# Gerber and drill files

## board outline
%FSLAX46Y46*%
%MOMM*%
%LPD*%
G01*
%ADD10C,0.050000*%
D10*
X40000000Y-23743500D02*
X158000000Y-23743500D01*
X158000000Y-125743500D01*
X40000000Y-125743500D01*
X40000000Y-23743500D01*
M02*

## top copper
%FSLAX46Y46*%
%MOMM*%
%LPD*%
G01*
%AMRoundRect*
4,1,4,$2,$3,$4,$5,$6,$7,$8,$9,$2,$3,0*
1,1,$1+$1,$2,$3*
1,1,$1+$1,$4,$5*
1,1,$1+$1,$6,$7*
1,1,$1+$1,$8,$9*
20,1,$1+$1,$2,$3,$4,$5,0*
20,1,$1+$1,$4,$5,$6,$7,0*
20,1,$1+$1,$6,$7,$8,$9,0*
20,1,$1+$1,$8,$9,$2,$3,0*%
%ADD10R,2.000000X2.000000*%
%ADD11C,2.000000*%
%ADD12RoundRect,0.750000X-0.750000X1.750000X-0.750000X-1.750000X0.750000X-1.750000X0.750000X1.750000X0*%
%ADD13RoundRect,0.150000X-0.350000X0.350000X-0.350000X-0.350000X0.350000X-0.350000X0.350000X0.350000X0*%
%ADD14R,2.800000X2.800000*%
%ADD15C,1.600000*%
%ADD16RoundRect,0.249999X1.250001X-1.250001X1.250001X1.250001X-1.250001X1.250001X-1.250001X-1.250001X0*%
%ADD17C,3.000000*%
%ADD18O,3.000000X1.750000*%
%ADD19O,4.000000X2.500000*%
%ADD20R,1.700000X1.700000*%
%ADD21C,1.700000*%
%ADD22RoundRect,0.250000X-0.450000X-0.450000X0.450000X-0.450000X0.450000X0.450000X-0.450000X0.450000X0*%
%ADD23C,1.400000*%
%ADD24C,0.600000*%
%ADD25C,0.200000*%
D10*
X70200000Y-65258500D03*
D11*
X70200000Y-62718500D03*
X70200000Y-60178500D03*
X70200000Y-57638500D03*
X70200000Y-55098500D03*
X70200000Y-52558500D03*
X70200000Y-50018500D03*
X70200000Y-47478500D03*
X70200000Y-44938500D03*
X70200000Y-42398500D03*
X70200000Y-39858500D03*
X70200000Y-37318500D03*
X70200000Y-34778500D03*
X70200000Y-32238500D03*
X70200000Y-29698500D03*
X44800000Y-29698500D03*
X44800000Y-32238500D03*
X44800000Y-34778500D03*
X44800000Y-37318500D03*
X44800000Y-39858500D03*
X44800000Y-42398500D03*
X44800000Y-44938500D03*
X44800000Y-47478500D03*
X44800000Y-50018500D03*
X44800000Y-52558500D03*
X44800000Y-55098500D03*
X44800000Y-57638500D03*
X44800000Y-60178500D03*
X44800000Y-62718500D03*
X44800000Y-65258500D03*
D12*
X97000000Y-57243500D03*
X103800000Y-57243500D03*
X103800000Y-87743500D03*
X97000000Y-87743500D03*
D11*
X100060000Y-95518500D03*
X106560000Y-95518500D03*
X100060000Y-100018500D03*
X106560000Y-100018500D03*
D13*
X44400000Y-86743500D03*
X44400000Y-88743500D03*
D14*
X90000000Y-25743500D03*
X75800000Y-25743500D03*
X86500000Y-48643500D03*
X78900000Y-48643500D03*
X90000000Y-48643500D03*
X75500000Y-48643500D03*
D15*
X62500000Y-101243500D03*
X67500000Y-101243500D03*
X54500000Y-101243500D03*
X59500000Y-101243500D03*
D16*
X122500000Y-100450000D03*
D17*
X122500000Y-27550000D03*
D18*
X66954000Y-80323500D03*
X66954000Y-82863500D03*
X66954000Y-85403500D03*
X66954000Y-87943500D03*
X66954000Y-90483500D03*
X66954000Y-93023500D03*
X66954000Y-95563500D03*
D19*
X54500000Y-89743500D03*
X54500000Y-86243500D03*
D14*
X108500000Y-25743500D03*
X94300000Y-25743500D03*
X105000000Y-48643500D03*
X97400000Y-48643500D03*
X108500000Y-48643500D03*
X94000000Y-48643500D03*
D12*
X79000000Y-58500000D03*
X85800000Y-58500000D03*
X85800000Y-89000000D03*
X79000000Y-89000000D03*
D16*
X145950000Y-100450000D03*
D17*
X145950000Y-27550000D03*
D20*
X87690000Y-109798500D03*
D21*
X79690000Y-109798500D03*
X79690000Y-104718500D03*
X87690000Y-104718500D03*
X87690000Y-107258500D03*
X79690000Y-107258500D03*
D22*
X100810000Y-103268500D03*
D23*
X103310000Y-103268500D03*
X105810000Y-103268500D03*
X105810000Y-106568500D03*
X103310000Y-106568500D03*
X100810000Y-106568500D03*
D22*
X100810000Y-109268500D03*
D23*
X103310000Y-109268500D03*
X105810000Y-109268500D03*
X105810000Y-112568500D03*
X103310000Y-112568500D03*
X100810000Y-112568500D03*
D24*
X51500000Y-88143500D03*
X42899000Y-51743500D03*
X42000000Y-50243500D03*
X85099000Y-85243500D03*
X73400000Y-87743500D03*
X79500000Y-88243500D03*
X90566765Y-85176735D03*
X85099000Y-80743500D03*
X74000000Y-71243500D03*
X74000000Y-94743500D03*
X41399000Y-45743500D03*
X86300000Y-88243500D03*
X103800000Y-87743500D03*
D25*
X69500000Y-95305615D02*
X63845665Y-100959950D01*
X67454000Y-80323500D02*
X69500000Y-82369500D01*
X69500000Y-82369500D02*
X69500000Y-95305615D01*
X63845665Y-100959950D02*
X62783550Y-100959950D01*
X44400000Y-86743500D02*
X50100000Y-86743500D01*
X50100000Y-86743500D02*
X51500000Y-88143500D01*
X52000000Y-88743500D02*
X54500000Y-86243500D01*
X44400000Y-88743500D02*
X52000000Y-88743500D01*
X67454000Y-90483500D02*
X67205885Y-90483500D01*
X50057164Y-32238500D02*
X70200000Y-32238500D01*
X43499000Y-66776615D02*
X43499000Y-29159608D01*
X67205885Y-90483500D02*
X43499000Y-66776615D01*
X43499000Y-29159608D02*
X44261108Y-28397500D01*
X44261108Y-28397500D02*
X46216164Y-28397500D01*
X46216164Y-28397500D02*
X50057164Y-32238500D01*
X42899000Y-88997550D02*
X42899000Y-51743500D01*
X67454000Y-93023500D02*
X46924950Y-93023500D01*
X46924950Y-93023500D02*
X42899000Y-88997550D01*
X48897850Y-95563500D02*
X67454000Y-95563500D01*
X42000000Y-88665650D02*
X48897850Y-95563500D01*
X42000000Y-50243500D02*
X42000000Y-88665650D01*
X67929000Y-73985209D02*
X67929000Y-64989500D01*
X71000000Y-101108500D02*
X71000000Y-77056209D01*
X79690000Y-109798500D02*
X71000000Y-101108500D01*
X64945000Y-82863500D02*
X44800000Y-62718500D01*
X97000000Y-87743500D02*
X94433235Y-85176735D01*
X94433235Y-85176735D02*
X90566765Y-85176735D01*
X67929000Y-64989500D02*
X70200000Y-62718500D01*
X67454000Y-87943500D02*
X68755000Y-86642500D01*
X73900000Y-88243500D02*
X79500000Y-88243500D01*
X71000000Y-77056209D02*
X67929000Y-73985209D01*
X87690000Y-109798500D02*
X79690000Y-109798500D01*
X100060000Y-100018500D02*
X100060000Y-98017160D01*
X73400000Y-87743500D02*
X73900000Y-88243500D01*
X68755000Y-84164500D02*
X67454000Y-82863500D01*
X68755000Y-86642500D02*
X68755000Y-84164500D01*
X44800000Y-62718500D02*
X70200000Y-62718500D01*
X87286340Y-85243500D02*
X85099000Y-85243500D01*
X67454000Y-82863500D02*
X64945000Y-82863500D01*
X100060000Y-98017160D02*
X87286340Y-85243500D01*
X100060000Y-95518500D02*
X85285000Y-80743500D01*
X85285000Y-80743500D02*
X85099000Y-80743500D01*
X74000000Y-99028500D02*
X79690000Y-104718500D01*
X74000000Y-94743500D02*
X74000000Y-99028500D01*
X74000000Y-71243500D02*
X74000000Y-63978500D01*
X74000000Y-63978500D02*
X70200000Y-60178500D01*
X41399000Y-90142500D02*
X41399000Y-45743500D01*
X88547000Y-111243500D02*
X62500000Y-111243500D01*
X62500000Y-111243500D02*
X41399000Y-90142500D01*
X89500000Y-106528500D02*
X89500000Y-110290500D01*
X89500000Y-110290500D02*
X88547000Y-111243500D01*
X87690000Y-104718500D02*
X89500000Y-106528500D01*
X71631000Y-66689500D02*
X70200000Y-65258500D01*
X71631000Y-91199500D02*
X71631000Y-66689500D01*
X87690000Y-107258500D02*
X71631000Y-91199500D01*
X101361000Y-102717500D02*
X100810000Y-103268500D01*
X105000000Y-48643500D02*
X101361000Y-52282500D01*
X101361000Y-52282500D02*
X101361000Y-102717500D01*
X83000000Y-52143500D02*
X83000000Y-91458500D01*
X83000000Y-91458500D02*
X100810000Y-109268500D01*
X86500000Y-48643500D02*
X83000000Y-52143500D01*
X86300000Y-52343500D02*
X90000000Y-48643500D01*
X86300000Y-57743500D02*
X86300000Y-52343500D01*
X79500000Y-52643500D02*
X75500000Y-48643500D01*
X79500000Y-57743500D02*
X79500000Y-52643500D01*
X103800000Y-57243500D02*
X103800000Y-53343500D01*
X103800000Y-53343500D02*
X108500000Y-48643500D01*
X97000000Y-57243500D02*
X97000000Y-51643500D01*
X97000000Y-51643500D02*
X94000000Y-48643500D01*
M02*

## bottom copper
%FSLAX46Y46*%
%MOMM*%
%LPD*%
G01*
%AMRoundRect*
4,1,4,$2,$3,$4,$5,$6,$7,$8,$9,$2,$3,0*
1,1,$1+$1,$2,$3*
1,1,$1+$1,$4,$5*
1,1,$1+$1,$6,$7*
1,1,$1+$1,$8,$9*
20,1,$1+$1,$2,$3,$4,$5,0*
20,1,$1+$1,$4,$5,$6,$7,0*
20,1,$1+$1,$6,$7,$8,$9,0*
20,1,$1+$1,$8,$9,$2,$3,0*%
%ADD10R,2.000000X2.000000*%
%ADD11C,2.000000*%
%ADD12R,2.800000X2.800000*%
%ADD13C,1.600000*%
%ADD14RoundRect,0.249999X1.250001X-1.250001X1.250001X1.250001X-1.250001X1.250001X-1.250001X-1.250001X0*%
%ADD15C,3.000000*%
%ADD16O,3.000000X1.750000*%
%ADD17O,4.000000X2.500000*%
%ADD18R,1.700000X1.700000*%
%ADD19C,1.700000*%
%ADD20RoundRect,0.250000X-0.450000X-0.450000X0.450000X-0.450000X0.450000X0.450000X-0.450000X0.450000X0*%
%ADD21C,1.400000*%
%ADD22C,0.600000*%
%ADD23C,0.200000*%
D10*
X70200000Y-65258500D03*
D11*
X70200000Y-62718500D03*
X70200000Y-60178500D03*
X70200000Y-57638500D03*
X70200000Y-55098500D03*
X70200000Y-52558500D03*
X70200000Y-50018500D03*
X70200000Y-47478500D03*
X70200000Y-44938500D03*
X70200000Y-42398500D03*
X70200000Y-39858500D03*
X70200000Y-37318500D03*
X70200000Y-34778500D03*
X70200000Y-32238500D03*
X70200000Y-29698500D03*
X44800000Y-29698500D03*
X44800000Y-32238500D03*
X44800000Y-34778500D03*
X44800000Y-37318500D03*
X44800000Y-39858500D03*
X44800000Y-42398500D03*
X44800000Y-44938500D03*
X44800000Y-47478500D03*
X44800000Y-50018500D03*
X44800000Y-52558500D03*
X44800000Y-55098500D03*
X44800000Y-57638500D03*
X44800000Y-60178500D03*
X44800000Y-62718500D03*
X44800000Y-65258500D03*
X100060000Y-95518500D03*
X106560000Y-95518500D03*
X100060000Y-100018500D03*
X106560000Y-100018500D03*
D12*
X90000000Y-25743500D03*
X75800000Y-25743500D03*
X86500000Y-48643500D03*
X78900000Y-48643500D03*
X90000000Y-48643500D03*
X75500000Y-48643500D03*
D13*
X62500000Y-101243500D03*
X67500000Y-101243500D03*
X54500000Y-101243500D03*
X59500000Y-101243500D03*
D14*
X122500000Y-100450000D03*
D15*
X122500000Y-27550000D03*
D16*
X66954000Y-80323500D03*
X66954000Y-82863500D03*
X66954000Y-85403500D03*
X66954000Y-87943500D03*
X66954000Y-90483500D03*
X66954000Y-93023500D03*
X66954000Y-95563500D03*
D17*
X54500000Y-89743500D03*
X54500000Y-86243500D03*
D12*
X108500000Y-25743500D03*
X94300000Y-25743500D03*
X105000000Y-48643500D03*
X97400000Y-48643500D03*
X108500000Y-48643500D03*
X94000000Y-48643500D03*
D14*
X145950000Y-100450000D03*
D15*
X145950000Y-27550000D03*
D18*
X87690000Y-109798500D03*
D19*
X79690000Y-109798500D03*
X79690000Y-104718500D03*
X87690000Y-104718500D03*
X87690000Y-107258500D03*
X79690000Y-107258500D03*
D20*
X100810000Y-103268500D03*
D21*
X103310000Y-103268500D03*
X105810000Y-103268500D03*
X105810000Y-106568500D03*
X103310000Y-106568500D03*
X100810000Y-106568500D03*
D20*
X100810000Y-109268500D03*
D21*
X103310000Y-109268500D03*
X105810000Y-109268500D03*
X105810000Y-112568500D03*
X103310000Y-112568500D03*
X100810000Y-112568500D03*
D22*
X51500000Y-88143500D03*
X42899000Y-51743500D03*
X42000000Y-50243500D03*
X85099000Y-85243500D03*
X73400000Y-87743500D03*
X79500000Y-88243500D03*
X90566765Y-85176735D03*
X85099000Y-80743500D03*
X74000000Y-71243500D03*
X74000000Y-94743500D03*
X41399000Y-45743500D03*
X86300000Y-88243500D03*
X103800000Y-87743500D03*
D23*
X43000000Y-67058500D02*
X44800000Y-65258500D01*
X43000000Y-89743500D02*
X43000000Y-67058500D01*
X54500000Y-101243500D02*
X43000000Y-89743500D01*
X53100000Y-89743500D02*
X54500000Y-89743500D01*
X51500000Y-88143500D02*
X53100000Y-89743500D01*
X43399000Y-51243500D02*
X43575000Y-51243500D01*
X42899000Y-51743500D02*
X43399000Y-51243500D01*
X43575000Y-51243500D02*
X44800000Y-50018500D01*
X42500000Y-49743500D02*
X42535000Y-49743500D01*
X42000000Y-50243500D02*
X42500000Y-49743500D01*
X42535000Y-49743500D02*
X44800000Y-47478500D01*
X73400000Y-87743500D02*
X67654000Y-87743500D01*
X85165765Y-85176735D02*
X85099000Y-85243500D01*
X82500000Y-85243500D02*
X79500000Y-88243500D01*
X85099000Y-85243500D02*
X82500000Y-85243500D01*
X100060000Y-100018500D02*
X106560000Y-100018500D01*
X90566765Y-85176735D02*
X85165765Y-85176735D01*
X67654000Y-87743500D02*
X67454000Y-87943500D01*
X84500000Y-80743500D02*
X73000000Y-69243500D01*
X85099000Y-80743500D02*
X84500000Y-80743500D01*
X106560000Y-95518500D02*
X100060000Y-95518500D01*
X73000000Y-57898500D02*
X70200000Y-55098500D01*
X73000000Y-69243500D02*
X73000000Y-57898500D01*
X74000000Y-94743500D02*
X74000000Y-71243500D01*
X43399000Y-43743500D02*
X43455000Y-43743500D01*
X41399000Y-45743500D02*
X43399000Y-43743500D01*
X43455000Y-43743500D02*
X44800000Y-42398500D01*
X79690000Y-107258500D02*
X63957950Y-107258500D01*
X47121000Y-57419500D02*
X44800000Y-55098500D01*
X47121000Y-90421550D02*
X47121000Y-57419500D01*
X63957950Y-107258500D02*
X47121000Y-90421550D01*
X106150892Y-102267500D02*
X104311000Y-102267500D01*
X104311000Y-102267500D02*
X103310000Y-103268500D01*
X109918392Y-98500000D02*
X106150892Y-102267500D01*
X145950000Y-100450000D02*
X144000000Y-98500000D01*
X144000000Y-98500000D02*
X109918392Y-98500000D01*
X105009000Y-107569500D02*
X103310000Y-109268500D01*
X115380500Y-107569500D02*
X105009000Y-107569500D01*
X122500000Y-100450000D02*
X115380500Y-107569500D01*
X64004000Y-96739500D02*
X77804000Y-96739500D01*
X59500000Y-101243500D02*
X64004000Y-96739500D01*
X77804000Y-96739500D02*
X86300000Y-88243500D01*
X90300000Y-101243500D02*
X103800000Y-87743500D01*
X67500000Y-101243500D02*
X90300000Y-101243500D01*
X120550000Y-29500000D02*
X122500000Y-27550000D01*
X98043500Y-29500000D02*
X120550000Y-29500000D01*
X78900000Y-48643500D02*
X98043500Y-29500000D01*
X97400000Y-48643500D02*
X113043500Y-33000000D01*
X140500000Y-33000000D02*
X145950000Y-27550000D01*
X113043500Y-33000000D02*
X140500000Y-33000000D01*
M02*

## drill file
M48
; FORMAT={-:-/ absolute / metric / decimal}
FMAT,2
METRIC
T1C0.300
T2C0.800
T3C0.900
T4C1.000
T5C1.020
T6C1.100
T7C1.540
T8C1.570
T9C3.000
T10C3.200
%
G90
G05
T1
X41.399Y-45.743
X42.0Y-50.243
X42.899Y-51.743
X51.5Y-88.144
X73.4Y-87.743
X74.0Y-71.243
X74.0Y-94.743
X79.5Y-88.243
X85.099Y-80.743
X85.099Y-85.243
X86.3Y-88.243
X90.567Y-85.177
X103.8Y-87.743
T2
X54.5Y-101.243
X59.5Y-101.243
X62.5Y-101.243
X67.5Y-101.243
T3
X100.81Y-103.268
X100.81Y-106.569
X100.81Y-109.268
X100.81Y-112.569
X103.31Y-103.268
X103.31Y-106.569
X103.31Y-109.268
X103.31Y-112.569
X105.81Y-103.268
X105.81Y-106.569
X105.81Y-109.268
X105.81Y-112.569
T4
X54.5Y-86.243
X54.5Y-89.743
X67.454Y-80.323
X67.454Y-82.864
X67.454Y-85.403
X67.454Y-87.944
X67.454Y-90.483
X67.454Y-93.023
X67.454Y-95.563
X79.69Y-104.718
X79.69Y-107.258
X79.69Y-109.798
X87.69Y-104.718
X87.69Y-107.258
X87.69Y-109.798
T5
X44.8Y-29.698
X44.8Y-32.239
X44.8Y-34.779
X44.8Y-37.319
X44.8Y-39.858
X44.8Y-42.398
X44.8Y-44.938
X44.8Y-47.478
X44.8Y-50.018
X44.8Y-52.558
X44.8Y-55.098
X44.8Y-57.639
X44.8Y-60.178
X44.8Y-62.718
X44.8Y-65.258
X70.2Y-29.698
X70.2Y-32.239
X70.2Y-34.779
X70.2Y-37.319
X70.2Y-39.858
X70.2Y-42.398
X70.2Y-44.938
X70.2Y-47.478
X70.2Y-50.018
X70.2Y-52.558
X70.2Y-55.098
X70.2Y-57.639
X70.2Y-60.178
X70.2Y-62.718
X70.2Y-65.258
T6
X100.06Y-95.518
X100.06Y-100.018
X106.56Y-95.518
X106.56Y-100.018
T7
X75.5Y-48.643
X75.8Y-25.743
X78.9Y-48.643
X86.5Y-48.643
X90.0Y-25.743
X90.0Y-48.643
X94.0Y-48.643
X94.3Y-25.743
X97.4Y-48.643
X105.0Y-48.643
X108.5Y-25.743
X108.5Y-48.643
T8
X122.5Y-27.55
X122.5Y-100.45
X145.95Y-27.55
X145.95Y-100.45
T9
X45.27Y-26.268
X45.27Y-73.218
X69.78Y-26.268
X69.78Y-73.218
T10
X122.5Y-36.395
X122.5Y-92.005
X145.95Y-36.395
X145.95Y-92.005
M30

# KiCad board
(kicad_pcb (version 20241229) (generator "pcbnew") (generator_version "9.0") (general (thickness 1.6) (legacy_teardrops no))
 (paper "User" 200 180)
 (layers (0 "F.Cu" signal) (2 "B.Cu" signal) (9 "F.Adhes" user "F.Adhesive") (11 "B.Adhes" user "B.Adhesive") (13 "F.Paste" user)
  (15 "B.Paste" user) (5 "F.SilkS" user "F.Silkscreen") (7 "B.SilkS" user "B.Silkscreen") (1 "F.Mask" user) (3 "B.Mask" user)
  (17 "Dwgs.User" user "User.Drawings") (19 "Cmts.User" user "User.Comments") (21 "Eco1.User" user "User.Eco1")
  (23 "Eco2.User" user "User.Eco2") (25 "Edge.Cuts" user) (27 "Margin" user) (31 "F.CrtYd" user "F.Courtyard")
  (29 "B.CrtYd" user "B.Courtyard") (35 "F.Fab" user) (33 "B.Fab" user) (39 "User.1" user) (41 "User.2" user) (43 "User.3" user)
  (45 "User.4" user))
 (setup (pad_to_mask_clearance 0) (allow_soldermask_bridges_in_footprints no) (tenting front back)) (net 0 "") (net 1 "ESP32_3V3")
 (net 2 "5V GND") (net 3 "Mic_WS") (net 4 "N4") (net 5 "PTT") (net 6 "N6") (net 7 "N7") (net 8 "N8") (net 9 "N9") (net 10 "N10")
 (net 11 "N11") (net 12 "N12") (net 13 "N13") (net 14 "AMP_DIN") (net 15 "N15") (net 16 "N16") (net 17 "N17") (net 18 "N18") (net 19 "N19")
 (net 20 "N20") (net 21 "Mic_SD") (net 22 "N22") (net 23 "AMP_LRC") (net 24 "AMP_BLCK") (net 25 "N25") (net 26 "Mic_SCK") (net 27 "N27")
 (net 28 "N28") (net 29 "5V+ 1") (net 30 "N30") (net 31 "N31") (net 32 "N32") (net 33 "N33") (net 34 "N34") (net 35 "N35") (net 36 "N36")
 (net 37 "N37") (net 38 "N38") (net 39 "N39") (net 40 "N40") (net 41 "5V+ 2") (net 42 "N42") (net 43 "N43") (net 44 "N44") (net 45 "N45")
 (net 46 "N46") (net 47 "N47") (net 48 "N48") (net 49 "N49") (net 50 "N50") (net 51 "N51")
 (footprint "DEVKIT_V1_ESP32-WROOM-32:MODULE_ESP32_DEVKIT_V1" (layer "F.Cu") (at 57.5 49.7435 180)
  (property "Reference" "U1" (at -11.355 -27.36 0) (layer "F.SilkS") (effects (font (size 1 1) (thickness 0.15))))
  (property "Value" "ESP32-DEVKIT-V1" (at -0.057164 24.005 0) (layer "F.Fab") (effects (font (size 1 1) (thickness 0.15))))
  (pad "" np_thru_hole circle (at -12.28 -23.475 180) (size 3 3) (drill 3) (layers "*.Cu" "*.Mask"))
  (pad "" np_thru_hole circle (at -12.28 23.475 180) (size 3 3) (drill 3) (layers "*.Cu" "*.Mask"))
  (pad "" np_thru_hole circle (at 12.23 -23.475 180) (size 3 3) (drill 3) (layers "*.Cu" "*.Mask"))
  (pad "" np_thru_hole circle (at 12.23 23.475 180) (size 3 3) (drill 3) (layers "*.Cu" "*.Mask"))
  (pad "1" thru_hole rect (at -12.7 -15.515 180) (size 2 2) (drill 1.02) (layers "*.Cu" "*.Mask") (remove_unused_layers no)
   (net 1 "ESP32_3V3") (solder_mask_margin 0.102))
  (pad "2" thru_hole circle (at -12.7 -12.975 180) (size 2 2) (drill 1.02) (layers "*.Cu" "*.Mask") (remove_unused_layers no)
   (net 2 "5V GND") (solder_mask_margin 0.102))
  (pad "3" thru_hole circle (at -12.7 -10.435 180) (size 2 2) (drill 1.02) (layers "*.Cu" "*.Mask") (remove_unused_layers no)
   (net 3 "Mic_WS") (solder_mask_margin 0.102))
  (pad "4" thru_hole circle (at -12.7 -7.895 180) (size 2 2) (drill 1.02) (layers "*.Cu" "*.Mask") (remove_unused_layers no) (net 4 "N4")
   (solder_mask_margin 0.102))
  (pad "5" thru_hole circle (at -12.7 -5.355 180) (size 2 2) (drill 1.02) (layers "*.Cu" "*.Mask") (remove_unused_layers no) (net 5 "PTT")
   (solder_mask_margin 0.102))
  (pad "6" thru_hole circle (at -12.7 -2.815 180) (size 2 2) (drill 1.02) (layers "*.Cu" "*.Mask") (remove_unused_layers no) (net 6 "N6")
   (solder_mask_margin 0.102))
  (pad "7" thru_hole circle (at -12.7 -0.275 180) (size 2 2) (drill 1.02) (layers "*.Cu" "*.Mask") (remove_unused_layers no) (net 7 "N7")
   (solder_mask_margin 0.102))
  (pad "8" thru_hole circle (at -12.7 2.265 180) (size 2 2) (drill 1.02) (layers "*.Cu" "*.Mask") (remove_unused_layers no) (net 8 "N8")
   (solder_mask_margin 0.102))
  (pad "9" thru_hole circle (at -12.7 4.805 180) (size 2 2) (drill 1.02) (layers "*.Cu" "*.Mask") (remove_unused_layers no) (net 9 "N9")
   (solder_mask_margin 0.102))
  (pad "10" thru_hole circle (at -12.7 7.345 180) (size 2 2) (drill 1.02) (layers "*.Cu" "*.Mask") (remove_unused_layers no) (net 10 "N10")
   (solder_mask_margin 0.102))
  (pad "11" thru_hole circle (at -12.7 9.885 180) (size 2 2) (drill 1.02) (layers "*.Cu" "*.Mask") (remove_unused_layers no) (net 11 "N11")
   (solder_mask_margin 0.102))
  (pad "12" thru_hole circle (at -12.7 12.425 180) (size 2 2) (drill 1.02) (layers "*.Cu" "*.Mask") (remove_unused_layers no) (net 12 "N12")
   (solder_mask_margin 0.102))
  (pad "13" thru_hole circle (at -12.7 14.965 180) (size 2 2) (drill 1.02) (layers "*.Cu" "*.Mask") (remove_unused_layers no) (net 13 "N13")
   (solder_mask_margin 0.102))
  (pad "14" thru_hole circle (at -12.7 17.505 180) (size 2 2) (drill 1.02) (layers "*.Cu" "*.Mask") (remove_unused_layers no)
   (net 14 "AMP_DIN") (solder_mask_margin 0.102))
  (pad "15" thru_hole circle (at -12.7 20.045 180) (size 2 2) (drill 1.02) (layers "*.Cu" "*.Mask") (remove_unused_layers no) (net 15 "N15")
   (solder_mask_margin 0.102))
  (pad "16" thru_hole circle (at 12.7 20.045 180) (size 2 2) (drill 1.02) (layers "*.Cu" "*.Mask") (remove_unused_layers no) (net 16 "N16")
   (solder_mask_margin 0.102))
  (pad "17" thru_hole circle (at 12.7 17.505 180) (size 2 2) (drill 1.02) (layers "*.Cu" "*.Mask") (remove_unused_layers no) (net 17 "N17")
   (solder_mask_margin 0.102))
  (pad "18" thru_hole circle (at 12.7 14.965 180) (size 2 2) (drill 1.02) (layers "*.Cu" "*.Mask") (remove_unused_layers no) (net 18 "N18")
   (solder_mask_margin 0.102))
  (pad "19" thru_hole circle (at 12.7 12.425 180) (size 2 2) (drill 1.02) (layers "*.Cu" "*.Mask") (remove_unused_layers no) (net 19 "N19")
   (solder_mask_margin 0.102))
  (pad "20" thru_hole circle (at 12.7 9.885 180) (size 2 2) (drill 1.02) (layers "*.Cu" "*.Mask") (remove_unused_layers no) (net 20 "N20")
   (solder_mask_margin 0.102))
  (pad "21" thru_hole circle (at 12.7 7.345 180) (size 2 2) (drill 1.02) (layers "*.Cu" "*.Mask") (remove_unused_layers no)
   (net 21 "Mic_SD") (solder_mask_margin 0.102))
  (pad "22" thru_hole circle (at 12.7 4.805 180) (size 2 2) (drill 1.02) (layers "*.Cu" "*.Mask") (remove_unused_layers no) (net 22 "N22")
   (solder_mask_margin 0.102))
  (pad "23" thru_hole circle (at 12.7 2.265 180) (size 2 2) (drill 1.02) (layers "*.Cu" "*.Mask") (remove_unused_layers no)
   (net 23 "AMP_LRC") (solder_mask_margin 0.102))
  (pad "24" thru_hole circle (at 12.7 -0.275 180) (size 2 2) (drill 1.02) (layers "*.Cu" "*.Mask") (remove_unused_layers no)
   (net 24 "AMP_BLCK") (solder_mask_margin 0.102))
  (pad "25" thru_hole circle (at 12.7 -2.815 180) (size 2 2) (drill 1.02) (layers "*.Cu" "*.Mask") (remove_unused_layers no) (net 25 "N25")
   (solder_mask_margin 0.102))
  (pad "26" thru_hole circle (at 12.7 -5.355 180) (size 2 2) (drill 1.02) (layers "*.Cu" "*.Mask") (remove_unused_layers no)
   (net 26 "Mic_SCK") (solder_mask_margin 0.102))
  (pad "27" thru_hole circle (at 12.7 -7.895 180) (size 2 2) (drill 1.02) (layers "*.Cu" "*.Mask") (remove_unused_layers no) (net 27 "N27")
   (solder_mask_margin 0.102))
  (pad "28" thru_hole circle (at 12.7 -10.435 180) (size 2 2) (drill 1.02) (layers "*.Cu" "*.Mask") (remove_unused_layers no) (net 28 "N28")
   (solder_mask_margin 0.102))
  (pad "29" thru_hole circle (at 12.7 -12.975 180) (size 2 2) (drill 1.02) (layers "*.Cu" "*.Mask") (remove_unused_layers no)
   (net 2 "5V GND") (solder_mask_margin 0.102))
  (pad "30" thru_hole circle (at 12.7 -15.515 180) (size 2 2) (drill 1.02) (layers "*.Cu" "*.Mask") (remove_unused_layers no)
   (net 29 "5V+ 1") (solder_mask_margin 0.102))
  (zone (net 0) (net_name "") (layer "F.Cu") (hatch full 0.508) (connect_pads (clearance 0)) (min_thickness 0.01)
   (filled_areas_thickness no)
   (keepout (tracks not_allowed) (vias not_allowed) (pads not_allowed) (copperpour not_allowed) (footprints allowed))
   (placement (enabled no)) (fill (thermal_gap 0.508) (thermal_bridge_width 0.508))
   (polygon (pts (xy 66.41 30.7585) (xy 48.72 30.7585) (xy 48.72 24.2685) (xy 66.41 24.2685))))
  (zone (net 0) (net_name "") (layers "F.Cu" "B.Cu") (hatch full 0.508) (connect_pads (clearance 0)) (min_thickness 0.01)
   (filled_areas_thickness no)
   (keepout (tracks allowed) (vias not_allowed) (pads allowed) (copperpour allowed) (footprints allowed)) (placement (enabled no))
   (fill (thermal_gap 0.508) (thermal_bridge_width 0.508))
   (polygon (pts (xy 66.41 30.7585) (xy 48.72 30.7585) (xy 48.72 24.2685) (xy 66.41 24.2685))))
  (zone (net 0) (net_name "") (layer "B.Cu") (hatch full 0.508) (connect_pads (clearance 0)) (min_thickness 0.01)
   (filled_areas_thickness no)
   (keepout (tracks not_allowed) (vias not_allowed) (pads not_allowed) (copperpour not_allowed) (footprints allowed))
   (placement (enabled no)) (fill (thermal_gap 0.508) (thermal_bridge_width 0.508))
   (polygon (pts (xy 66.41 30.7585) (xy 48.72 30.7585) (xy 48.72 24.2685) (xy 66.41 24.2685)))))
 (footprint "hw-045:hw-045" (layer "F.Cu") (at 99.9 72.2435 -90)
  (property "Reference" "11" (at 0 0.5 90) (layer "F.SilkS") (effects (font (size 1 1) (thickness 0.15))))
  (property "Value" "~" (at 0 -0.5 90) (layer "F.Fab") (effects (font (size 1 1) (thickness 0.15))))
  (pad "1" smd roundrect (at -15 2.9 270) (size 5 3) (layers "F.Cu" "F.Mask" "F.Paste") (roundrect_rratio 0.25) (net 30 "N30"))
  (pad "2" smd roundrect (at -15 -3.9 270) (size 5 3) (layers "F.Cu" "F.Mask" "F.Paste") (roundrect_rratio 0.25) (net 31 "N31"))
  (pad "3" smd roundrect (at 15.5 -3.9 270) (size 5 3) (layers "F.Cu" "F.Mask" "F.Paste") (roundrect_rratio 0.25) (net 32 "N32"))
  (pad "4" smd roundrect (at 15.5 2.9 270) (size 5 3) (layers "F.Cu" "F.Mask" "F.Paste") (roundrect_rratio 0.25) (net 2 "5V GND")))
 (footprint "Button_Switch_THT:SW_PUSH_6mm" (layer "F.Cu") (at 100.06 95.5185)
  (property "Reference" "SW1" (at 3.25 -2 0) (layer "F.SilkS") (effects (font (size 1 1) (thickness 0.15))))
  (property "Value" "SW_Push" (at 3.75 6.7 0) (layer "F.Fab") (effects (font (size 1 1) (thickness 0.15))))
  (pad "1" thru_hole circle (at 0 0 90) (size 2 2) (drill 1.1) (layers "*.Cu" "*.Mask") (remove_unused_layers no) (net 5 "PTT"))
  (pad "1" thru_hole circle (at 6.5 0 90) (size 2 2) (drill 1.1) (layers "*.Cu" "*.Mask") (remove_unused_layers no) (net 5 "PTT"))
  (pad "2" thru_hole circle (at 0 4.5 90) (size 2 2) (drill 1.1) (layers "*.Cu" "*.Mask") (remove_unused_layers no) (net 2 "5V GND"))
  (pad "2" thru_hole circle (at 6.5 4.5 90) (size 2 2) (drill 1.1) (layers "*.Cu" "*.Mask") (remove_unused_layers no) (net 2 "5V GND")))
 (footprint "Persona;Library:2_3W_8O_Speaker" (layer "F.Cu") (at 45.4 87.7435 -90)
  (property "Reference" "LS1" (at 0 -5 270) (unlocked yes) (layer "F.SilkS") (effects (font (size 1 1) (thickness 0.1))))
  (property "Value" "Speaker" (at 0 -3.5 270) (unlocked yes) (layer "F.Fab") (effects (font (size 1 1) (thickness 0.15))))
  (pad "1" smd roundrect (at -1 1 270) (size 1 1) (layers "F.Cu" "F.Mask" "F.Paste") (roundrect_rratio 0.15) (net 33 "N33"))
  (pad "2" smd roundrect (at 1 1 270) (size 1 1) (layers "F.Cu" "F.Mask" "F.Paste") (roundrect_rratio 0.15) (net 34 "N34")))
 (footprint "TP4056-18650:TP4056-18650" (layer "F.Cu") (at 91.7 24.0435 -90)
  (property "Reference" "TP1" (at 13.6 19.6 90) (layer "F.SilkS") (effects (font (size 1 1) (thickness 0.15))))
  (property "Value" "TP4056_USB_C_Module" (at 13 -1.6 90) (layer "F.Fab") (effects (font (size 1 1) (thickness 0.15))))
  (pad "1" thru_hole rect (at 1.7 1.7 270) (size 2.8 2.8) (drill 1.54) (layers "*.Cu" "*.Mask") (remove_unused_layers no) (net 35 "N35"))
  (pad "2" thru_hole rect (at 1.7 15.9 270) (size 2.8 2.8) (drill 1.54) (layers "*.Cu" "*.Mask") (remove_unused_layers no) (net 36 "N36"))
  (pad "3" thru_hole rect (at 24.6 5.2 270) (size 2.8 2.8) (drill 1.54) (layers "*.Cu" "*.Mask") (remove_unused_layers no) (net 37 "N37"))
  (pad "4" thru_hole rect (at 24.6 12.8 270) (size 2.8 2.8) (drill 1.54) (layers "*.Cu" "*.Mask") (remove_unused_layers no) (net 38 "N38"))
  (pad "5" thru_hole rect (at 24.6 1.7 270) (size 2.8 2.8) (drill 1.54) (layers "*.Cu" "*.Mask") (remove_unused_layers no) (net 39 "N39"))
  (pad "6" thru_hole rect (at 24.6 16.2 270) (size 2.8 2.8) (drill 1.54) (layers "*.Cu" "*.Mask") (remove_unused_layers no) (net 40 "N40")))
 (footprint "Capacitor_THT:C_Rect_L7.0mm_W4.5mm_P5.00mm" (layer "F.Cu") (at 62.5 101.2435)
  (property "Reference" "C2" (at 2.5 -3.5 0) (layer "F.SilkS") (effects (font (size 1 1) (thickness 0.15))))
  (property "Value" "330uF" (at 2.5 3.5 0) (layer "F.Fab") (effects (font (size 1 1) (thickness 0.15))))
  (pad "1" thru_hole circle (at 0 0) (size 1.6 1.6) (drill 0.8) (layers "*.Cu" "*.Mask") (remove_unused_layers no) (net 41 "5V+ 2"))
  (pad "2" thru_hole circle (at 5 0) (size 1.6 1.6) (drill 0.8) (layers "*.Cu" "*.Mask") (remove_unused_layers no) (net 32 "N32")))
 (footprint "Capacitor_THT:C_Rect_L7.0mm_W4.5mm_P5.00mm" (layer "F.Cu") (at 54.5 101.2435)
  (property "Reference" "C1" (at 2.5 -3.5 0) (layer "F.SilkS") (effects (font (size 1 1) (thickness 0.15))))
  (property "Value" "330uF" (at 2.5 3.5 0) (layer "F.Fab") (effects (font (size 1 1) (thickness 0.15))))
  (pad "1" thru_hole circle (at 0 0) (size 1.6 1.6) (drill 0.8) (layers "*.Cu" "*.Mask") (remove_unused_layers no) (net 29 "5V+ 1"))
  (pad "2" thru_hole circle (at 5 0) (size 1.6 1.6) (drill 0.8) (layers "*.Cu" "*.Mask") (remove_unused_layers no) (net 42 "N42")))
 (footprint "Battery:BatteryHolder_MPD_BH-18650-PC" (layer "F.Cu") (at 122.5 100.45 90)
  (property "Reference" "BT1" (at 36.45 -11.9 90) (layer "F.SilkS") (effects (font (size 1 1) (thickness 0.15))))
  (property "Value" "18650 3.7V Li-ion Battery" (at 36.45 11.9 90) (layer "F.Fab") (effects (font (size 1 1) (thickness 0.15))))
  (pad "" np_thru_hole circle (at 8.445 0 90) (size 3.2 3.2) (drill 3.2) (layers "*.Cu" "*.Mask"))
  (pad "" np_thru_hole circle (at 64.055 0 90) (size 3.2 3.2) (drill 3.2) (layers "*.Cu" "*.Mask"))
  (pad "1" thru_hole roundrect (at 0 0 90) (size 3 3) (drill 1.57) (layers "*.Cu" "*.Mask") (remove_unused_layers no)
   (roundrect_rratio 0.083333) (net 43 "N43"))
  (pad "2" thru_hole circle (at 72.9 0 90) (size 3 3) (drill 1.57) (layers "*.Cu" "*.Mask") (remove_unused_layers no) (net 38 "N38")))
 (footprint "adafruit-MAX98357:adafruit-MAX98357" (layer "F.Cu") (at 60.547 87.8235 90)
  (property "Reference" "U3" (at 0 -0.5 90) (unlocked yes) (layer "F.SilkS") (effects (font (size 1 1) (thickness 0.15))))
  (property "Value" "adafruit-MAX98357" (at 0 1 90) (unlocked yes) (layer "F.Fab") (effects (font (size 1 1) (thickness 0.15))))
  (pad "1" thru_hole oval (at 7.5 6.907) (size 3 1.75) (drill 1 (offset -0.5 0)) (layers "*.Cu" "*.Mask") (remove_unused_layers no)
   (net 41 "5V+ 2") (solder_mask_margin 0.0508))
  (pad "2" thru_hole oval (at 4.96 6.907) (size 3 1.75) (drill 1 (offset -0.5 0)) (layers "*.Cu" "*.Mask") (remove_unused_layers no)
   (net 2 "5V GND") (solder_mask_margin 0.0508))
  (pad "3" thru_hole oval (at 2.42 6.907) (size 3 1.75) (drill 1 (offset -0.5 0)) (layers "*.Cu" "*.Mask") (remove_unused_layers no)
   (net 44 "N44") (solder_mask_margin 0.0508))
  (pad "4" thru_hole oval (at -0.12 6.907) (size 3 1.75) (drill 1 (offset -0.5 0)) (layers "*.Cu" "*.Mask") (remove_unused_layers no)
   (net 2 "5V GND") (solder_mask_margin 0.0508))
  (pad "5" thru_hole oval (at -2.66 6.907) (size 3 1.75) (drill 1 (offset -0.5 0)) (layers "*.Cu" "*.Mask") (remove_unused_layers no)
   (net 14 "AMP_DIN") (solder_mask_margin 0.0508))
  (pad "6" thru_hole oval (at -5.2 6.907) (size 3 1.75) (drill 1 (offset -0.5 0)) (layers "*.Cu" "*.Mask") (remove_unused_layers no)
   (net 24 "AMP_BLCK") (solder_mask_margin 0.0508))
  (pad "7" thru_hole oval (at -7.74 6.907) (size 3 1.75) (drill 1 (offset -0.5 0)) (layers "*.Cu" "*.Mask") (remove_unused_layers no)
   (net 23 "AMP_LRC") (solder_mask_margin 0.0508))
  (pad "8" thru_hole oval (at -1.92 -6.047 270) (size 2.5 4) (drill 1) (layers "*.Cu" "*.Mask") (remove_unused_layers no) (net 33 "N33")
   (solder_mask_margin 0.0508))
  (pad "9" thru_hole oval (at 1.58 -6.047 270) (size 2.5 4) (drill 1) (layers "*.Cu" "*.Mask") (remove_unused_layers no) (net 34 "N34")
   (solder_mask_margin 0.0508)))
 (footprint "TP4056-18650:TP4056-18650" (layer "F.Cu") (at 110.2 24.0435 -90)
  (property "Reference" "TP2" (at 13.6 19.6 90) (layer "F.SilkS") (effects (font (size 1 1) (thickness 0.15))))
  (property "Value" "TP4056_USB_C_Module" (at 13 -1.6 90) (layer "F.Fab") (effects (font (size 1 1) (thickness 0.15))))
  (pad "1" thru_hole rect (at 1.7 1.7 270) (size 2.8 2.8) (drill 1.54) (layers "*.Cu" "*.Mask") (remove_unused_layers no) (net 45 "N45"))
  (pad "2" thru_hole rect (at 1.7 15.9 270) (size 2.8 2.8) (drill 1.54) (layers "*.Cu" "*.Mask") (remove_unused_layers no) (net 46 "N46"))
  (pad "3" thru_hole rect (at 24.6 5.2 270) (size 2.8 2.8) (drill 1.54) (layers "*.Cu" "*.Mask") (remove_unused_layers no) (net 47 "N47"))
  (pad "4" thru_hole rect (at 24.6 12.8 270) (size 2.8 2.8) (drill 1.54) (layers "*.Cu" "*.Mask") (remove_unused_layers no) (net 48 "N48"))
  (pad "5" thru_hole rect (at 24.6 1.7 270) (size 2.8 2.8) (drill 1.54) (layers "*.Cu" "*.Mask") (remove_unused_layers no) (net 31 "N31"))
  (pad "6" thru_hole rect (at 24.6 16.2 270) (size 2.8 2.8) (drill 1.54) (layers "*.Cu" "*.Mask") (remove_unused_layers no) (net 30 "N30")))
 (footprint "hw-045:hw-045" (layer "F.Cu") (at 81.9 73.5 -90)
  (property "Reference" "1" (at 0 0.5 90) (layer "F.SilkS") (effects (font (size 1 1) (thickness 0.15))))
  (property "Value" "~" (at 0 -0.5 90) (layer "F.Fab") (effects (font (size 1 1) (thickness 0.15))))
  (pad "1" smd roundrect (at -15 2.9 270) (size 5 3) (layers "F.Cu" "F.Mask" "F.Paste") (roundrect_rratio 0.25) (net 40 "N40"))
  (pad "2" smd roundrect (at -15 -3.9 270) (size 5 3) (layers "F.Cu" "F.Mask" "F.Paste") (roundrect_rratio 0.25) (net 39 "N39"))
  (pad "3" smd roundrect (at 15.5 -3.9 270) (size 5 3) (layers "F.Cu" "F.Mask" "F.Paste") (roundrect_rratio 0.25) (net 42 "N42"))
  (pad "4" smd roundrect (at 15.5 2.9 270) (size 5 3) (layers "F.Cu" "F.Mask" "F.Paste") (roundrect_rratio 0.25) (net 2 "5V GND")))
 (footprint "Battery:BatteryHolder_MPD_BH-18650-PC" (layer "F.Cu") (at 145.95 100.45 90)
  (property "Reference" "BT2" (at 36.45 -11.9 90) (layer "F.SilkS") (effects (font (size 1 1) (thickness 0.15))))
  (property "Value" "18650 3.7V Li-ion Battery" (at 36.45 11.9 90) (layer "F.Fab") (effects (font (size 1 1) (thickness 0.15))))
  (pad "" np_thru_hole circle (at 8.445 0 90) (size 3.2 3.2) (drill 3.2) (layers "*.Cu" "*.Mask"))
  (pad "" np_thru_hole circle (at 64.055 0 90) (size 3.2 3.2) (drill 3.2) (layers "*.Cu" "*.Mask"))
  (pad "1" thru_hole roundrect (at 0 0 90) (size 3 3) (drill 1.57) (layers "*.Cu" "*.Mask") (remove_unused_layers no)
   (roundrect_rratio 0.083333) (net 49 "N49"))
  (pad "2" thru_hole circle (at 72.9 0 90) (size 3 3) (drill 1.57) (layers "*.Cu" "*.Mask") (remove_unused_layers no) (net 48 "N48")))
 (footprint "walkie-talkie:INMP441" (layer "F.Cu") (at 83.5 114.2435 180)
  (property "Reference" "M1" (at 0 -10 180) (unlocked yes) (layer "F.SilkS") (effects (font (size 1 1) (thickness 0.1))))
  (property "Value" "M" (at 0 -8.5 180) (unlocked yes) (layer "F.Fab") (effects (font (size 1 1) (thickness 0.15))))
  (pad "GND" thru_hole rect (at -4.19 4.445 180) (size 1.7 1.7) (drill 1) (layers "*.Cu" "*.Mask") (remove_unused_layers no)
   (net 2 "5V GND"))
  (pad "L/R" thru_hole circle (at 3.81 4.445 180) (size 1.7 1.7) (drill 1) (layers "*.Cu" "*.Mask") (remove_unused_layers no)
   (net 2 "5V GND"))
  (pad "SCK" thru_hole circle (at 3.81 9.525 180) (size 1.7 1.7) (drill 1) (layers "*.Cu" "*.Mask") (remove_unused_layers no)
   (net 3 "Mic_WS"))
  (pad "SD" thru_hole circle (at -4.19 9.525 180) (size 1.7 1.7) (drill 1) (layers "*.Cu" "*.Mask") (remove_unused_layers no)
   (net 21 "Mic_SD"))
  (pad "VDD" thru_hole circle (at -4.19 6.985 180) (size 1.7 1.7) (drill 1) (layers "*.Cu" "*.Mask") (remove_unused_layers no)
   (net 1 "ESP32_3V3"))
  (pad "WS" thru_hole circle (at 3.81 6.985 180) (size 1.7 1.7) (drill 1) (layers "*.Cu" "*.Mask") (remove_unused_layers no)
   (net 26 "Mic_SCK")))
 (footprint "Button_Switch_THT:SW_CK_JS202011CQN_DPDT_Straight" (layer "F.Cu") (at 100.81 103.2685)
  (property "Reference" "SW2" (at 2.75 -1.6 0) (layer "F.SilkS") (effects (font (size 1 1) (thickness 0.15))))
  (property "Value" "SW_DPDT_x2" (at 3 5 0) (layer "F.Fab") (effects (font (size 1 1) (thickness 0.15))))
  (pad "1" thru_hole roundrect (at 0 0) (size 1.4 1.4) (drill 0.9) (layers "*.Cu" "*.Mask") (remove_unused_layers no)
   (roundrect_rratio 0.1785714286) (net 47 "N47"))
  (pad "2" thru_hole circle (at 2.5 0) (size 1.4 1.4) (drill 0.9) (layers "*.Cu" "*.Mask") (remove_unused_layers no) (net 49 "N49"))
  (pad "3" thru_hole circle (at 5 0) (size 1.4 1.4) (drill 0.9) (layers "*.Cu" "*.Mask") (remove_unused_layers no) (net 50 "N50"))
  (pad "4" thru_hole circle (at 5 3.3) (size 1.4 1.4) (drill 0.9) (layers "*.Cu" "*.Mask") (remove_unused_layers no))
  (pad "5" thru_hole circle (at 2.5 3.3) (size 1.4 1.4) (drill 0.9) (layers "*.Cu" "*.Mask") (remove_unused_layers no))
  (pad "6" thru_hole circle (at 0 3.3) (size 1.4 1.4) (drill 0.9) (layers "*.Cu" "*.Mask") (remove_unused_layers no)))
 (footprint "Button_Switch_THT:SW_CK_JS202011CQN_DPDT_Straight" (layer "F.Cu") (at 100.81 109.2685)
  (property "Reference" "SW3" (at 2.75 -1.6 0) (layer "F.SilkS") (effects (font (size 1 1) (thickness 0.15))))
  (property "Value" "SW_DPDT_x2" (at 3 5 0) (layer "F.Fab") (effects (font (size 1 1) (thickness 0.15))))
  (pad "1" thru_hole roundrect (at 0 0) (size 1.4 1.4) (drill 0.9) (layers "*.Cu" "*.Mask") (remove_unused_layers no)
   (roundrect_rratio 0.1785714286) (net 37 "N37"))
  (pad "2" thru_hole circle (at 2.5 0) (size 1.4 1.4) (drill 0.9) (layers "*.Cu" "*.Mask") (remove_unused_layers no) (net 43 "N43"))
  (pad "3" thru_hole circle (at 5 0) (size 1.4 1.4) (drill 0.9) (layers "*.Cu" "*.Mask") (remove_unused_layers no) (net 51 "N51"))
  (pad "4" thru_hole circle (at 5 3.3) (size 1.4 1.4) (drill 0.9) (layers "*.Cu" "*.Mask") (remove_unused_layers no))
  (pad "5" thru_hole circle (at 2.5 3.3) (size 1.4 1.4) (drill 0.9) (layers "*.Cu" "*.Mask") (remove_unused_layers no))
  (pad "6" thru_hole circle (at 0 3.3) (size 1.4 1.4) (drill 0.9) (layers "*.Cu" "*.Mask") (remove_unused_layers no)))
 (gr_rect (start 40 23.7435) (end 158 125.7435) (stroke (width 0.05) (type default)) (fill no) (layer "Edge.Cuts"))
 (segment (start 43 67.0585) (end 44.8 65.2585) (width 0.2) (layer "B.Cu") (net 29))
 (segment (start 43 89.7435) (end 43 67.0585) (width 0.2) (layer "B.Cu") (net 29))
 (segment (start 54.5 101.2435) (end 43 89.7435) (width 0.2) (layer "B.Cu") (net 29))
 (segment (start 69.5 95.305615) (end 63.845665 100.95995) (width 0.2) (layer "F.Cu") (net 41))
 (segment (start 67.454 80.3235) (end 69.5 82.3695) (width 0.2) (layer "F.Cu") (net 41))
 (segment (start 69.5 82.3695) (end 69.5 95.305615) (width 0.2) (layer "F.Cu") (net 41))
 (segment (start 63.845665 100.95995) (end 62.78355 100.95995) (width 0.2) (layer "F.Cu") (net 41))
 (segment (start 44.4 86.7435) (end 50.1 86.7435) (width 0.2) (layer "F.Cu") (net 33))
 (segment (start 50.1 86.7435) (end 51.5 88.1435) (width 0.2) (layer "F.Cu") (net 33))
 (via (at 51.5 88.1435) (size 0.6) (drill 0.3) (layers "F.Cu" "B.Cu") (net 33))
 (segment (start 53.1 89.7435) (end 54.5 89.7435) (width 0.2) (layer "B.Cu") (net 33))
 (segment (start 51.5 88.1435) (end 53.1 89.7435) (width 0.2) (layer "B.Cu") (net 33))
 (segment (start 52 88.7435) (end 54.5 86.2435) (width 0.2) (layer "F.Cu") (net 34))
 (segment (start 44.4 88.7435) (end 52 88.7435) (width 0.2) (layer "F.Cu") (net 34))
 (segment (start 67.454 90.4835) (end 67.205885 90.4835) (width 0.2) (layer "F.Cu") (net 14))
 (segment (start 50.057164 32.2385) (end 70.2 32.2385) (width 0.2) (layer "F.Cu") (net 14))
 (segment (start 43.499 66.776615) (end 43.499 29.159608) (width 0.2) (layer "F.Cu") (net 14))
 (segment (start 67.205885 90.4835) (end 43.499 66.776615) (width 0.2) (layer "F.Cu") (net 14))
 (segment (start 43.499 29.159608) (end 44.261108 28.3975) (width 0.2) (layer "F.Cu") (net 14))
 (segment (start 44.261108 28.3975) (end 46.216164 28.3975) (width 0.2) (layer "F.Cu") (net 14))
 (segment (start 46.216164 28.3975) (end 50.057164 32.2385) (width 0.2) (layer "F.Cu") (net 14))
 (segment (start 42.899 88.99755) (end 42.899 51.7435) (width 0.2) (layer "F.Cu") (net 24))
 (segment (start 67.454 93.0235) (end 46.92495 93.0235) (width 0.2) (layer "F.Cu") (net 24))
 (segment (start 46.92495 93.0235) (end 42.899 88.99755) (width 0.2) (layer "F.Cu") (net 24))
 (via (at 42.899 51.7435) (size 0.6) (drill 0.3) (layers "F.Cu" "B.Cu") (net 24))
 (segment (start 43.399 51.2435) (end 43.575 51.2435) (width 0.2) (layer "B.Cu") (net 24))
 (segment (start 42.899 51.7435) (end 43.399 51.2435) (width 0.2) (layer "B.Cu") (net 24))
 (segment (start 43.575 51.2435) (end 44.8 50.0185) (width 0.2) (layer "B.Cu") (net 24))
 (segment (start 48.89785 95.5635) (end 67.454 95.5635) (width 0.2) (layer "F.Cu") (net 23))
 (segment (start 42 88.66565) (end 48.89785 95.5635) (width 0.2) (layer "F.Cu") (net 23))
 (segment (start 42 50.2435) (end 42 88.66565) (width 0.2) (layer "F.Cu") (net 23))
 (via (at 42 50.2435) (size 0.6) (drill 0.3) (layers "F.Cu" "B.Cu") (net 23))
 (segment (start 42.5 49.7435) (end 42.535 49.7435) (width 0.2) (layer "B.Cu") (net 23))
 (segment (start 42 50.2435) (end 42.5 49.7435) (width 0.2) (layer "B.Cu") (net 23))
 (segment (start 42.535 49.7435) (end 44.8 47.4785) (width 0.2) (layer "B.Cu") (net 23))
 (segment (start 67.929 73.985209) (end 67.929 64.9895) (width 0.2) (layer "F.Cu") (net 2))
 (segment (start 71 101.1085) (end 71 77.056209) (width 0.2) (layer "F.Cu") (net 2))
 (segment (start 79.69 109.7985) (end 71 101.1085) (width 0.2) (layer "F.Cu") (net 2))
 (segment (start 64.945 82.8635) (end 44.8 62.7185) (width 0.2) (layer "F.Cu") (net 2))
 (segment (start 97 87.7435) (end 94.433235 85.176735) (width 0.2) (layer "F.Cu") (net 2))
 (segment (start 94.433235 85.176735) (end 90.566765 85.176735) (width 0.2) (layer "F.Cu") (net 2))
 (segment (start 67.929 64.9895) (end 70.2 62.7185) (width 0.2) (layer "F.Cu") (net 2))
 (segment (start 67.454 87.9435) (end 68.755 86.6425) (width 0.2) (layer "F.Cu") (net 2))
 (segment (start 73.9 88.2435) (end 79.5 88.2435) (width 0.2) (layer "F.Cu") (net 2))
 (segment (start 71 77.056209) (end 67.929 73.985209) (width 0.2) (layer "F.Cu") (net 2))
 (segment (start 87.69 109.7985) (end 79.69 109.7985) (width 0.2) (layer "F.Cu") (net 2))
 (segment (start 100.06 100.0185) (end 100.06 98.01716) (width 0.2) (layer "F.Cu") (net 2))
 (segment (start 73.4 87.7435) (end 73.9 88.2435) (width 0.2) (layer "F.Cu") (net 2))
 (segment (start 68.755 84.1645) (end 67.454 82.8635) (width 0.2) (layer "F.Cu") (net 2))
 (segment (start 68.755 86.6425) (end 68.755 84.1645) (width 0.2) (layer "F.Cu") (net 2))
 (segment (start 44.8 62.7185) (end 70.2 62.7185) (width 0.2) (layer "F.Cu") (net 2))
 (segment (start 87.28634 85.2435) (end 85.099 85.2435) (width 0.2) (layer "F.Cu") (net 2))
 (segment (start 67.454 82.8635) (end 64.945 82.8635) (width 0.2) (layer "F.Cu") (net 2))
 (segment (start 100.06 98.01716) (end 87.28634 85.2435) (width 0.2) (layer "F.Cu") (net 2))
 (via (at 85.099 85.2435) (size 0.6) (drill 0.3) (layers "F.Cu" "B.Cu") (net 2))
 (via (at 73.4 87.7435) (size 0.6) (drill 0.3) (layers "F.Cu" "B.Cu") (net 2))
 (via (at 79.5 88.2435) (size 0.6) (drill 0.3) (layers "F.Cu" "B.Cu") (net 2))
 (via (at 90.566765 85.176735) (size 0.6) (drill 0.3) (layers "F.Cu" "B.Cu") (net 2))
 (segment (start 73.4 87.7435) (end 67.654 87.7435) (width 0.2) (layer "B.Cu") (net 2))
 (segment (start 85.165765 85.176735) (end 85.099 85.2435) (width 0.2) (layer "B.Cu") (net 2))
 (segment (start 82.5 85.2435) (end 79.5 88.2435) (width 0.2) (layer "B.Cu") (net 2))
 (segment (start 85.099 85.2435) (end 82.5 85.2435) (width 0.2) (layer "B.Cu") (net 2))
 (segment (start 100.06 100.0185) (end 106.56 100.0185) (width 0.2) (layer "B.Cu") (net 2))
 (segment (start 90.566765 85.176735) (end 85.165765 85.176735) (width 0.2) (layer "B.Cu") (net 2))
 (segment (start 67.654 87.7435) (end 67.454 87.9435) (width 0.2) (layer "B.Cu") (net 2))
 (segment (start 100.06 95.5185) (end 85.285 80.7435) (width 0.2) (layer "F.Cu") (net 5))
 (segment (start 85.285 80.7435) (end 85.099 80.7435) (width 0.2) (layer "F.Cu") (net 5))
 (via (at 85.099 80.7435) (size 0.6) (drill 0.3) (layers "F.Cu" "B.Cu") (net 5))
 (segment (start 84.5 80.7435) (end 73 69.2435) (width 0.2) (layer "B.Cu") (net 5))
 (segment (start 85.099 80.7435) (end 84.5 80.7435) (width 0.2) (layer "B.Cu") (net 5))
 (segment (start 106.56 95.5185) (end 100.06 95.5185) (width 0.2) (layer "B.Cu") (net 5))
 (segment (start 73 57.8985) (end 70.2 55.0985) (width 0.2) (layer "B.Cu") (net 5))
 (segment (start 73 69.2435) (end 73 57.8985) (width 0.2) (layer "B.Cu") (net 5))
 (segment (start 74 99.0285) (end 79.69 104.7185) (width 0.2) (layer "F.Cu") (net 3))
 (segment (start 74 94.7435) (end 74 99.0285) (width 0.2) (layer "F.Cu") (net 3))
 (segment (start 74 71.2435) (end 74 63.9785) (width 0.2) (layer "F.Cu") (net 3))
 (segment (start 74 63.9785) (end 70.2 60.1785) (width 0.2) (layer "F.Cu") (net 3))
 (via (at 74 71.2435) (size 0.6) (drill 0.3) (layers "F.Cu" "B.Cu") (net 3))
 (via (at 74 94.7435) (size 0.6) (drill 0.3) (layers "F.Cu" "B.Cu") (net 3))
 (segment (start 74 94.7435) (end 74 71.2435) (width 0.2) (layer "B.Cu") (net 3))
 (segment (start 41.399 90.1425) (end 41.399 45.7435) (width 0.2) (layer "F.Cu") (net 21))
 (segment (start 88.547 111.2435) (end 62.5 111.2435) (width 0.2) (layer "F.Cu") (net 21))
 (segment (start 62.5 111.2435) (end 41.399 90.1425) (width 0.2) (layer "F.Cu") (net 21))
 (segment (start 89.5 106.5285) (end 89.5 110.2905) (width 0.2) (layer "F.Cu") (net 21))
 (segment (start 89.5 110.2905) (end 88.547 111.2435) (width 0.2) (layer "F.Cu") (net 21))
 (segment (start 87.69 104.7185) (end 89.5 106.5285) (width 0.2) (layer "F.Cu") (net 21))
 (via (at 41.399 45.7435) (size 0.6) (drill 0.3) (layers "F.Cu" "B.Cu") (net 21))
 (segment (start 43.399 43.7435) (end 43.455 43.7435) (width 0.2) (layer "B.Cu") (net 21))
 (segment (start 41.399 45.7435) (end 43.399 43.7435) (width 0.2) (layer "B.Cu") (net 21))
 (segment (start 43.455 43.7435) (end 44.8 42.3985) (width 0.2) (layer "B.Cu") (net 21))
 (segment (start 71.631 66.6895) (end 70.2 65.2585) (width 0.2) (layer "F.Cu") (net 1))
 (segment (start 71.631 91.1995) (end 71.631 66.6895) (width 0.2) (layer "F.Cu") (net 1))
 (segment (start 87.69 107.2585) (end 71.631 91.1995) (width 0.2) (layer "F.Cu") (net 1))
 (segment (start 79.69 107.2585) (end 63.95795 107.2585) (width 0.2) (layer "B.Cu") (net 26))
 (segment (start 47.121 57.4195) (end 44.8 55.0985) (width 0.2) (layer "B.Cu") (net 26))
 (segment (start 47.121 90.42155) (end 47.121 57.4195) (width 0.2) (layer "B.Cu") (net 26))
 (segment (start 63.95795 107.2585) (end 47.121 90.42155) (width 0.2) (layer "B.Cu") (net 26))
 (segment (start 106.150892 102.2675) (end 104.311 102.2675) (width 0.2) (layer "B.Cu") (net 49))
 (segment (start 104.311 102.2675) (end 103.31 103.2685) (width 0.2) (layer "B.Cu") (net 49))
 (segment (start 109.918392 98.5) (end 106.150892 102.2675) (width 0.2) (layer "B.Cu") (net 49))
 (segment (start 145.95 100.45) (end 144 98.5) (width 0.2) (layer "B.Cu") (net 49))
 (segment (start 144 98.5) (end 109.918392 98.5) (width 0.2) (layer "B.Cu") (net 49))
 (segment (start 101.361 102.7175) (end 100.81 103.2685) (width 0.2) (layer "F.Cu") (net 47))
 (segment (start 105 48.6435) (end 101.361 52.2825) (width 0.2) (layer "F.Cu") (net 47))
 (segment (start 101.361 52.2825) (end 101.361 102.7175) (width 0.2) (layer "F.Cu") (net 47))
 (segment (start 105.009 107.5695) (end 103.31 109.2685) (width 0.2) (layer "B.Cu") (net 43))
 (segment (start 115.3805 107.5695) (end 105.009 107.5695) (width 0.2) (layer "B.Cu") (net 43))
 (segment (start 122.5 100.45) (end 115.3805 107.5695) (width 0.2) (layer "B.Cu") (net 43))
 (segment (start 83 52.1435) (end 83 91.4585) (width 0.2) (layer "F.Cu") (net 37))
 (segment (start 83 91.4585) (end 100.81 109.2685) (width 0.2) (layer "F.Cu") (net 37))
 (segment (start 86.5 48.6435) (end 83 52.1435) (width 0.2) (layer "F.Cu") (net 37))
 (segment (start 86.3 52.3435) (end 90 48.6435) (width 0.2) (layer "F.Cu") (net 39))
 (segment (start 86.3 57.7435) (end 86.3 52.3435) (width 0.2) (layer "F.Cu") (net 39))
 (via (at 86.3 88.2435) (size 0.6) (drill 0.3) (layers "F.Cu" "B.Cu") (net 42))
 (segment (start 64.004 96.7395) (end 77.804 96.7395) (width 0.2) (layer "B.Cu") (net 42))
 (segment (start 59.5 101.2435) (end 64.004 96.7395) (width 0.2) (layer "B.Cu") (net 42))
 (segment (start 77.804 96.7395) (end 86.3 88.2435) (width 0.2) (layer "B.Cu") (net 42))
 (segment (start 79.5 52.6435) (end 75.5 48.6435) (width 0.2) (layer "F.Cu") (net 40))
 (segment (start 79.5 57.7435) (end 79.5 52.6435) (width 0.2) (layer "F.Cu") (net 40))
 (segment (start 103.8 57.2435) (end 103.8 53.3435) (width 0.2) (layer "F.Cu") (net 31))
 (segment (start 103.8 53.3435) (end 108.5 48.6435) (width 0.2) (layer "F.Cu") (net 31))
 (segment (start 97 57.2435) (end 97 51.6435) (width 0.2) (layer "F.Cu") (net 30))
 (segment (start 97 51.6435) (end 94 48.6435) (width 0.2) (layer "F.Cu") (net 30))
 (via (at 103.8 87.7435) (size 0.6) (drill 0.3) (layers "F.Cu" "B.Cu") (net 32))
 (segment (start 90.3 101.2435) (end 103.8 87.7435) (width 0.2) (layer "B.Cu") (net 32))
 (segment (start 67.5 101.2435) (end 90.3 101.2435) (width 0.2) (layer "B.Cu") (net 32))
 (segment (start 120.55 29.5) (end 122.5 27.55) (width 0.2) (layer "B.Cu") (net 38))
 (segment (start 98.0435 29.5) (end 120.55 29.5) (width 0.2) (layer "B.Cu") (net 38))
 (segment (start 78.9 48.6435) (end 98.0435 29.5) (width 0.2) (layer "B.Cu") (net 38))
 (segment (start 97.4 48.6435) (end 113.0435 33) (width 0.2) (layer "B.Cu") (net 48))
 (segment (start 140.5 33) (end 145.95 27.55) (width 0.2) (layer "B.Cu") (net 48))
 (segment (start 113.0435 33) (end 140.5 33) (width 0.2) (layer "B.Cu") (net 48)))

